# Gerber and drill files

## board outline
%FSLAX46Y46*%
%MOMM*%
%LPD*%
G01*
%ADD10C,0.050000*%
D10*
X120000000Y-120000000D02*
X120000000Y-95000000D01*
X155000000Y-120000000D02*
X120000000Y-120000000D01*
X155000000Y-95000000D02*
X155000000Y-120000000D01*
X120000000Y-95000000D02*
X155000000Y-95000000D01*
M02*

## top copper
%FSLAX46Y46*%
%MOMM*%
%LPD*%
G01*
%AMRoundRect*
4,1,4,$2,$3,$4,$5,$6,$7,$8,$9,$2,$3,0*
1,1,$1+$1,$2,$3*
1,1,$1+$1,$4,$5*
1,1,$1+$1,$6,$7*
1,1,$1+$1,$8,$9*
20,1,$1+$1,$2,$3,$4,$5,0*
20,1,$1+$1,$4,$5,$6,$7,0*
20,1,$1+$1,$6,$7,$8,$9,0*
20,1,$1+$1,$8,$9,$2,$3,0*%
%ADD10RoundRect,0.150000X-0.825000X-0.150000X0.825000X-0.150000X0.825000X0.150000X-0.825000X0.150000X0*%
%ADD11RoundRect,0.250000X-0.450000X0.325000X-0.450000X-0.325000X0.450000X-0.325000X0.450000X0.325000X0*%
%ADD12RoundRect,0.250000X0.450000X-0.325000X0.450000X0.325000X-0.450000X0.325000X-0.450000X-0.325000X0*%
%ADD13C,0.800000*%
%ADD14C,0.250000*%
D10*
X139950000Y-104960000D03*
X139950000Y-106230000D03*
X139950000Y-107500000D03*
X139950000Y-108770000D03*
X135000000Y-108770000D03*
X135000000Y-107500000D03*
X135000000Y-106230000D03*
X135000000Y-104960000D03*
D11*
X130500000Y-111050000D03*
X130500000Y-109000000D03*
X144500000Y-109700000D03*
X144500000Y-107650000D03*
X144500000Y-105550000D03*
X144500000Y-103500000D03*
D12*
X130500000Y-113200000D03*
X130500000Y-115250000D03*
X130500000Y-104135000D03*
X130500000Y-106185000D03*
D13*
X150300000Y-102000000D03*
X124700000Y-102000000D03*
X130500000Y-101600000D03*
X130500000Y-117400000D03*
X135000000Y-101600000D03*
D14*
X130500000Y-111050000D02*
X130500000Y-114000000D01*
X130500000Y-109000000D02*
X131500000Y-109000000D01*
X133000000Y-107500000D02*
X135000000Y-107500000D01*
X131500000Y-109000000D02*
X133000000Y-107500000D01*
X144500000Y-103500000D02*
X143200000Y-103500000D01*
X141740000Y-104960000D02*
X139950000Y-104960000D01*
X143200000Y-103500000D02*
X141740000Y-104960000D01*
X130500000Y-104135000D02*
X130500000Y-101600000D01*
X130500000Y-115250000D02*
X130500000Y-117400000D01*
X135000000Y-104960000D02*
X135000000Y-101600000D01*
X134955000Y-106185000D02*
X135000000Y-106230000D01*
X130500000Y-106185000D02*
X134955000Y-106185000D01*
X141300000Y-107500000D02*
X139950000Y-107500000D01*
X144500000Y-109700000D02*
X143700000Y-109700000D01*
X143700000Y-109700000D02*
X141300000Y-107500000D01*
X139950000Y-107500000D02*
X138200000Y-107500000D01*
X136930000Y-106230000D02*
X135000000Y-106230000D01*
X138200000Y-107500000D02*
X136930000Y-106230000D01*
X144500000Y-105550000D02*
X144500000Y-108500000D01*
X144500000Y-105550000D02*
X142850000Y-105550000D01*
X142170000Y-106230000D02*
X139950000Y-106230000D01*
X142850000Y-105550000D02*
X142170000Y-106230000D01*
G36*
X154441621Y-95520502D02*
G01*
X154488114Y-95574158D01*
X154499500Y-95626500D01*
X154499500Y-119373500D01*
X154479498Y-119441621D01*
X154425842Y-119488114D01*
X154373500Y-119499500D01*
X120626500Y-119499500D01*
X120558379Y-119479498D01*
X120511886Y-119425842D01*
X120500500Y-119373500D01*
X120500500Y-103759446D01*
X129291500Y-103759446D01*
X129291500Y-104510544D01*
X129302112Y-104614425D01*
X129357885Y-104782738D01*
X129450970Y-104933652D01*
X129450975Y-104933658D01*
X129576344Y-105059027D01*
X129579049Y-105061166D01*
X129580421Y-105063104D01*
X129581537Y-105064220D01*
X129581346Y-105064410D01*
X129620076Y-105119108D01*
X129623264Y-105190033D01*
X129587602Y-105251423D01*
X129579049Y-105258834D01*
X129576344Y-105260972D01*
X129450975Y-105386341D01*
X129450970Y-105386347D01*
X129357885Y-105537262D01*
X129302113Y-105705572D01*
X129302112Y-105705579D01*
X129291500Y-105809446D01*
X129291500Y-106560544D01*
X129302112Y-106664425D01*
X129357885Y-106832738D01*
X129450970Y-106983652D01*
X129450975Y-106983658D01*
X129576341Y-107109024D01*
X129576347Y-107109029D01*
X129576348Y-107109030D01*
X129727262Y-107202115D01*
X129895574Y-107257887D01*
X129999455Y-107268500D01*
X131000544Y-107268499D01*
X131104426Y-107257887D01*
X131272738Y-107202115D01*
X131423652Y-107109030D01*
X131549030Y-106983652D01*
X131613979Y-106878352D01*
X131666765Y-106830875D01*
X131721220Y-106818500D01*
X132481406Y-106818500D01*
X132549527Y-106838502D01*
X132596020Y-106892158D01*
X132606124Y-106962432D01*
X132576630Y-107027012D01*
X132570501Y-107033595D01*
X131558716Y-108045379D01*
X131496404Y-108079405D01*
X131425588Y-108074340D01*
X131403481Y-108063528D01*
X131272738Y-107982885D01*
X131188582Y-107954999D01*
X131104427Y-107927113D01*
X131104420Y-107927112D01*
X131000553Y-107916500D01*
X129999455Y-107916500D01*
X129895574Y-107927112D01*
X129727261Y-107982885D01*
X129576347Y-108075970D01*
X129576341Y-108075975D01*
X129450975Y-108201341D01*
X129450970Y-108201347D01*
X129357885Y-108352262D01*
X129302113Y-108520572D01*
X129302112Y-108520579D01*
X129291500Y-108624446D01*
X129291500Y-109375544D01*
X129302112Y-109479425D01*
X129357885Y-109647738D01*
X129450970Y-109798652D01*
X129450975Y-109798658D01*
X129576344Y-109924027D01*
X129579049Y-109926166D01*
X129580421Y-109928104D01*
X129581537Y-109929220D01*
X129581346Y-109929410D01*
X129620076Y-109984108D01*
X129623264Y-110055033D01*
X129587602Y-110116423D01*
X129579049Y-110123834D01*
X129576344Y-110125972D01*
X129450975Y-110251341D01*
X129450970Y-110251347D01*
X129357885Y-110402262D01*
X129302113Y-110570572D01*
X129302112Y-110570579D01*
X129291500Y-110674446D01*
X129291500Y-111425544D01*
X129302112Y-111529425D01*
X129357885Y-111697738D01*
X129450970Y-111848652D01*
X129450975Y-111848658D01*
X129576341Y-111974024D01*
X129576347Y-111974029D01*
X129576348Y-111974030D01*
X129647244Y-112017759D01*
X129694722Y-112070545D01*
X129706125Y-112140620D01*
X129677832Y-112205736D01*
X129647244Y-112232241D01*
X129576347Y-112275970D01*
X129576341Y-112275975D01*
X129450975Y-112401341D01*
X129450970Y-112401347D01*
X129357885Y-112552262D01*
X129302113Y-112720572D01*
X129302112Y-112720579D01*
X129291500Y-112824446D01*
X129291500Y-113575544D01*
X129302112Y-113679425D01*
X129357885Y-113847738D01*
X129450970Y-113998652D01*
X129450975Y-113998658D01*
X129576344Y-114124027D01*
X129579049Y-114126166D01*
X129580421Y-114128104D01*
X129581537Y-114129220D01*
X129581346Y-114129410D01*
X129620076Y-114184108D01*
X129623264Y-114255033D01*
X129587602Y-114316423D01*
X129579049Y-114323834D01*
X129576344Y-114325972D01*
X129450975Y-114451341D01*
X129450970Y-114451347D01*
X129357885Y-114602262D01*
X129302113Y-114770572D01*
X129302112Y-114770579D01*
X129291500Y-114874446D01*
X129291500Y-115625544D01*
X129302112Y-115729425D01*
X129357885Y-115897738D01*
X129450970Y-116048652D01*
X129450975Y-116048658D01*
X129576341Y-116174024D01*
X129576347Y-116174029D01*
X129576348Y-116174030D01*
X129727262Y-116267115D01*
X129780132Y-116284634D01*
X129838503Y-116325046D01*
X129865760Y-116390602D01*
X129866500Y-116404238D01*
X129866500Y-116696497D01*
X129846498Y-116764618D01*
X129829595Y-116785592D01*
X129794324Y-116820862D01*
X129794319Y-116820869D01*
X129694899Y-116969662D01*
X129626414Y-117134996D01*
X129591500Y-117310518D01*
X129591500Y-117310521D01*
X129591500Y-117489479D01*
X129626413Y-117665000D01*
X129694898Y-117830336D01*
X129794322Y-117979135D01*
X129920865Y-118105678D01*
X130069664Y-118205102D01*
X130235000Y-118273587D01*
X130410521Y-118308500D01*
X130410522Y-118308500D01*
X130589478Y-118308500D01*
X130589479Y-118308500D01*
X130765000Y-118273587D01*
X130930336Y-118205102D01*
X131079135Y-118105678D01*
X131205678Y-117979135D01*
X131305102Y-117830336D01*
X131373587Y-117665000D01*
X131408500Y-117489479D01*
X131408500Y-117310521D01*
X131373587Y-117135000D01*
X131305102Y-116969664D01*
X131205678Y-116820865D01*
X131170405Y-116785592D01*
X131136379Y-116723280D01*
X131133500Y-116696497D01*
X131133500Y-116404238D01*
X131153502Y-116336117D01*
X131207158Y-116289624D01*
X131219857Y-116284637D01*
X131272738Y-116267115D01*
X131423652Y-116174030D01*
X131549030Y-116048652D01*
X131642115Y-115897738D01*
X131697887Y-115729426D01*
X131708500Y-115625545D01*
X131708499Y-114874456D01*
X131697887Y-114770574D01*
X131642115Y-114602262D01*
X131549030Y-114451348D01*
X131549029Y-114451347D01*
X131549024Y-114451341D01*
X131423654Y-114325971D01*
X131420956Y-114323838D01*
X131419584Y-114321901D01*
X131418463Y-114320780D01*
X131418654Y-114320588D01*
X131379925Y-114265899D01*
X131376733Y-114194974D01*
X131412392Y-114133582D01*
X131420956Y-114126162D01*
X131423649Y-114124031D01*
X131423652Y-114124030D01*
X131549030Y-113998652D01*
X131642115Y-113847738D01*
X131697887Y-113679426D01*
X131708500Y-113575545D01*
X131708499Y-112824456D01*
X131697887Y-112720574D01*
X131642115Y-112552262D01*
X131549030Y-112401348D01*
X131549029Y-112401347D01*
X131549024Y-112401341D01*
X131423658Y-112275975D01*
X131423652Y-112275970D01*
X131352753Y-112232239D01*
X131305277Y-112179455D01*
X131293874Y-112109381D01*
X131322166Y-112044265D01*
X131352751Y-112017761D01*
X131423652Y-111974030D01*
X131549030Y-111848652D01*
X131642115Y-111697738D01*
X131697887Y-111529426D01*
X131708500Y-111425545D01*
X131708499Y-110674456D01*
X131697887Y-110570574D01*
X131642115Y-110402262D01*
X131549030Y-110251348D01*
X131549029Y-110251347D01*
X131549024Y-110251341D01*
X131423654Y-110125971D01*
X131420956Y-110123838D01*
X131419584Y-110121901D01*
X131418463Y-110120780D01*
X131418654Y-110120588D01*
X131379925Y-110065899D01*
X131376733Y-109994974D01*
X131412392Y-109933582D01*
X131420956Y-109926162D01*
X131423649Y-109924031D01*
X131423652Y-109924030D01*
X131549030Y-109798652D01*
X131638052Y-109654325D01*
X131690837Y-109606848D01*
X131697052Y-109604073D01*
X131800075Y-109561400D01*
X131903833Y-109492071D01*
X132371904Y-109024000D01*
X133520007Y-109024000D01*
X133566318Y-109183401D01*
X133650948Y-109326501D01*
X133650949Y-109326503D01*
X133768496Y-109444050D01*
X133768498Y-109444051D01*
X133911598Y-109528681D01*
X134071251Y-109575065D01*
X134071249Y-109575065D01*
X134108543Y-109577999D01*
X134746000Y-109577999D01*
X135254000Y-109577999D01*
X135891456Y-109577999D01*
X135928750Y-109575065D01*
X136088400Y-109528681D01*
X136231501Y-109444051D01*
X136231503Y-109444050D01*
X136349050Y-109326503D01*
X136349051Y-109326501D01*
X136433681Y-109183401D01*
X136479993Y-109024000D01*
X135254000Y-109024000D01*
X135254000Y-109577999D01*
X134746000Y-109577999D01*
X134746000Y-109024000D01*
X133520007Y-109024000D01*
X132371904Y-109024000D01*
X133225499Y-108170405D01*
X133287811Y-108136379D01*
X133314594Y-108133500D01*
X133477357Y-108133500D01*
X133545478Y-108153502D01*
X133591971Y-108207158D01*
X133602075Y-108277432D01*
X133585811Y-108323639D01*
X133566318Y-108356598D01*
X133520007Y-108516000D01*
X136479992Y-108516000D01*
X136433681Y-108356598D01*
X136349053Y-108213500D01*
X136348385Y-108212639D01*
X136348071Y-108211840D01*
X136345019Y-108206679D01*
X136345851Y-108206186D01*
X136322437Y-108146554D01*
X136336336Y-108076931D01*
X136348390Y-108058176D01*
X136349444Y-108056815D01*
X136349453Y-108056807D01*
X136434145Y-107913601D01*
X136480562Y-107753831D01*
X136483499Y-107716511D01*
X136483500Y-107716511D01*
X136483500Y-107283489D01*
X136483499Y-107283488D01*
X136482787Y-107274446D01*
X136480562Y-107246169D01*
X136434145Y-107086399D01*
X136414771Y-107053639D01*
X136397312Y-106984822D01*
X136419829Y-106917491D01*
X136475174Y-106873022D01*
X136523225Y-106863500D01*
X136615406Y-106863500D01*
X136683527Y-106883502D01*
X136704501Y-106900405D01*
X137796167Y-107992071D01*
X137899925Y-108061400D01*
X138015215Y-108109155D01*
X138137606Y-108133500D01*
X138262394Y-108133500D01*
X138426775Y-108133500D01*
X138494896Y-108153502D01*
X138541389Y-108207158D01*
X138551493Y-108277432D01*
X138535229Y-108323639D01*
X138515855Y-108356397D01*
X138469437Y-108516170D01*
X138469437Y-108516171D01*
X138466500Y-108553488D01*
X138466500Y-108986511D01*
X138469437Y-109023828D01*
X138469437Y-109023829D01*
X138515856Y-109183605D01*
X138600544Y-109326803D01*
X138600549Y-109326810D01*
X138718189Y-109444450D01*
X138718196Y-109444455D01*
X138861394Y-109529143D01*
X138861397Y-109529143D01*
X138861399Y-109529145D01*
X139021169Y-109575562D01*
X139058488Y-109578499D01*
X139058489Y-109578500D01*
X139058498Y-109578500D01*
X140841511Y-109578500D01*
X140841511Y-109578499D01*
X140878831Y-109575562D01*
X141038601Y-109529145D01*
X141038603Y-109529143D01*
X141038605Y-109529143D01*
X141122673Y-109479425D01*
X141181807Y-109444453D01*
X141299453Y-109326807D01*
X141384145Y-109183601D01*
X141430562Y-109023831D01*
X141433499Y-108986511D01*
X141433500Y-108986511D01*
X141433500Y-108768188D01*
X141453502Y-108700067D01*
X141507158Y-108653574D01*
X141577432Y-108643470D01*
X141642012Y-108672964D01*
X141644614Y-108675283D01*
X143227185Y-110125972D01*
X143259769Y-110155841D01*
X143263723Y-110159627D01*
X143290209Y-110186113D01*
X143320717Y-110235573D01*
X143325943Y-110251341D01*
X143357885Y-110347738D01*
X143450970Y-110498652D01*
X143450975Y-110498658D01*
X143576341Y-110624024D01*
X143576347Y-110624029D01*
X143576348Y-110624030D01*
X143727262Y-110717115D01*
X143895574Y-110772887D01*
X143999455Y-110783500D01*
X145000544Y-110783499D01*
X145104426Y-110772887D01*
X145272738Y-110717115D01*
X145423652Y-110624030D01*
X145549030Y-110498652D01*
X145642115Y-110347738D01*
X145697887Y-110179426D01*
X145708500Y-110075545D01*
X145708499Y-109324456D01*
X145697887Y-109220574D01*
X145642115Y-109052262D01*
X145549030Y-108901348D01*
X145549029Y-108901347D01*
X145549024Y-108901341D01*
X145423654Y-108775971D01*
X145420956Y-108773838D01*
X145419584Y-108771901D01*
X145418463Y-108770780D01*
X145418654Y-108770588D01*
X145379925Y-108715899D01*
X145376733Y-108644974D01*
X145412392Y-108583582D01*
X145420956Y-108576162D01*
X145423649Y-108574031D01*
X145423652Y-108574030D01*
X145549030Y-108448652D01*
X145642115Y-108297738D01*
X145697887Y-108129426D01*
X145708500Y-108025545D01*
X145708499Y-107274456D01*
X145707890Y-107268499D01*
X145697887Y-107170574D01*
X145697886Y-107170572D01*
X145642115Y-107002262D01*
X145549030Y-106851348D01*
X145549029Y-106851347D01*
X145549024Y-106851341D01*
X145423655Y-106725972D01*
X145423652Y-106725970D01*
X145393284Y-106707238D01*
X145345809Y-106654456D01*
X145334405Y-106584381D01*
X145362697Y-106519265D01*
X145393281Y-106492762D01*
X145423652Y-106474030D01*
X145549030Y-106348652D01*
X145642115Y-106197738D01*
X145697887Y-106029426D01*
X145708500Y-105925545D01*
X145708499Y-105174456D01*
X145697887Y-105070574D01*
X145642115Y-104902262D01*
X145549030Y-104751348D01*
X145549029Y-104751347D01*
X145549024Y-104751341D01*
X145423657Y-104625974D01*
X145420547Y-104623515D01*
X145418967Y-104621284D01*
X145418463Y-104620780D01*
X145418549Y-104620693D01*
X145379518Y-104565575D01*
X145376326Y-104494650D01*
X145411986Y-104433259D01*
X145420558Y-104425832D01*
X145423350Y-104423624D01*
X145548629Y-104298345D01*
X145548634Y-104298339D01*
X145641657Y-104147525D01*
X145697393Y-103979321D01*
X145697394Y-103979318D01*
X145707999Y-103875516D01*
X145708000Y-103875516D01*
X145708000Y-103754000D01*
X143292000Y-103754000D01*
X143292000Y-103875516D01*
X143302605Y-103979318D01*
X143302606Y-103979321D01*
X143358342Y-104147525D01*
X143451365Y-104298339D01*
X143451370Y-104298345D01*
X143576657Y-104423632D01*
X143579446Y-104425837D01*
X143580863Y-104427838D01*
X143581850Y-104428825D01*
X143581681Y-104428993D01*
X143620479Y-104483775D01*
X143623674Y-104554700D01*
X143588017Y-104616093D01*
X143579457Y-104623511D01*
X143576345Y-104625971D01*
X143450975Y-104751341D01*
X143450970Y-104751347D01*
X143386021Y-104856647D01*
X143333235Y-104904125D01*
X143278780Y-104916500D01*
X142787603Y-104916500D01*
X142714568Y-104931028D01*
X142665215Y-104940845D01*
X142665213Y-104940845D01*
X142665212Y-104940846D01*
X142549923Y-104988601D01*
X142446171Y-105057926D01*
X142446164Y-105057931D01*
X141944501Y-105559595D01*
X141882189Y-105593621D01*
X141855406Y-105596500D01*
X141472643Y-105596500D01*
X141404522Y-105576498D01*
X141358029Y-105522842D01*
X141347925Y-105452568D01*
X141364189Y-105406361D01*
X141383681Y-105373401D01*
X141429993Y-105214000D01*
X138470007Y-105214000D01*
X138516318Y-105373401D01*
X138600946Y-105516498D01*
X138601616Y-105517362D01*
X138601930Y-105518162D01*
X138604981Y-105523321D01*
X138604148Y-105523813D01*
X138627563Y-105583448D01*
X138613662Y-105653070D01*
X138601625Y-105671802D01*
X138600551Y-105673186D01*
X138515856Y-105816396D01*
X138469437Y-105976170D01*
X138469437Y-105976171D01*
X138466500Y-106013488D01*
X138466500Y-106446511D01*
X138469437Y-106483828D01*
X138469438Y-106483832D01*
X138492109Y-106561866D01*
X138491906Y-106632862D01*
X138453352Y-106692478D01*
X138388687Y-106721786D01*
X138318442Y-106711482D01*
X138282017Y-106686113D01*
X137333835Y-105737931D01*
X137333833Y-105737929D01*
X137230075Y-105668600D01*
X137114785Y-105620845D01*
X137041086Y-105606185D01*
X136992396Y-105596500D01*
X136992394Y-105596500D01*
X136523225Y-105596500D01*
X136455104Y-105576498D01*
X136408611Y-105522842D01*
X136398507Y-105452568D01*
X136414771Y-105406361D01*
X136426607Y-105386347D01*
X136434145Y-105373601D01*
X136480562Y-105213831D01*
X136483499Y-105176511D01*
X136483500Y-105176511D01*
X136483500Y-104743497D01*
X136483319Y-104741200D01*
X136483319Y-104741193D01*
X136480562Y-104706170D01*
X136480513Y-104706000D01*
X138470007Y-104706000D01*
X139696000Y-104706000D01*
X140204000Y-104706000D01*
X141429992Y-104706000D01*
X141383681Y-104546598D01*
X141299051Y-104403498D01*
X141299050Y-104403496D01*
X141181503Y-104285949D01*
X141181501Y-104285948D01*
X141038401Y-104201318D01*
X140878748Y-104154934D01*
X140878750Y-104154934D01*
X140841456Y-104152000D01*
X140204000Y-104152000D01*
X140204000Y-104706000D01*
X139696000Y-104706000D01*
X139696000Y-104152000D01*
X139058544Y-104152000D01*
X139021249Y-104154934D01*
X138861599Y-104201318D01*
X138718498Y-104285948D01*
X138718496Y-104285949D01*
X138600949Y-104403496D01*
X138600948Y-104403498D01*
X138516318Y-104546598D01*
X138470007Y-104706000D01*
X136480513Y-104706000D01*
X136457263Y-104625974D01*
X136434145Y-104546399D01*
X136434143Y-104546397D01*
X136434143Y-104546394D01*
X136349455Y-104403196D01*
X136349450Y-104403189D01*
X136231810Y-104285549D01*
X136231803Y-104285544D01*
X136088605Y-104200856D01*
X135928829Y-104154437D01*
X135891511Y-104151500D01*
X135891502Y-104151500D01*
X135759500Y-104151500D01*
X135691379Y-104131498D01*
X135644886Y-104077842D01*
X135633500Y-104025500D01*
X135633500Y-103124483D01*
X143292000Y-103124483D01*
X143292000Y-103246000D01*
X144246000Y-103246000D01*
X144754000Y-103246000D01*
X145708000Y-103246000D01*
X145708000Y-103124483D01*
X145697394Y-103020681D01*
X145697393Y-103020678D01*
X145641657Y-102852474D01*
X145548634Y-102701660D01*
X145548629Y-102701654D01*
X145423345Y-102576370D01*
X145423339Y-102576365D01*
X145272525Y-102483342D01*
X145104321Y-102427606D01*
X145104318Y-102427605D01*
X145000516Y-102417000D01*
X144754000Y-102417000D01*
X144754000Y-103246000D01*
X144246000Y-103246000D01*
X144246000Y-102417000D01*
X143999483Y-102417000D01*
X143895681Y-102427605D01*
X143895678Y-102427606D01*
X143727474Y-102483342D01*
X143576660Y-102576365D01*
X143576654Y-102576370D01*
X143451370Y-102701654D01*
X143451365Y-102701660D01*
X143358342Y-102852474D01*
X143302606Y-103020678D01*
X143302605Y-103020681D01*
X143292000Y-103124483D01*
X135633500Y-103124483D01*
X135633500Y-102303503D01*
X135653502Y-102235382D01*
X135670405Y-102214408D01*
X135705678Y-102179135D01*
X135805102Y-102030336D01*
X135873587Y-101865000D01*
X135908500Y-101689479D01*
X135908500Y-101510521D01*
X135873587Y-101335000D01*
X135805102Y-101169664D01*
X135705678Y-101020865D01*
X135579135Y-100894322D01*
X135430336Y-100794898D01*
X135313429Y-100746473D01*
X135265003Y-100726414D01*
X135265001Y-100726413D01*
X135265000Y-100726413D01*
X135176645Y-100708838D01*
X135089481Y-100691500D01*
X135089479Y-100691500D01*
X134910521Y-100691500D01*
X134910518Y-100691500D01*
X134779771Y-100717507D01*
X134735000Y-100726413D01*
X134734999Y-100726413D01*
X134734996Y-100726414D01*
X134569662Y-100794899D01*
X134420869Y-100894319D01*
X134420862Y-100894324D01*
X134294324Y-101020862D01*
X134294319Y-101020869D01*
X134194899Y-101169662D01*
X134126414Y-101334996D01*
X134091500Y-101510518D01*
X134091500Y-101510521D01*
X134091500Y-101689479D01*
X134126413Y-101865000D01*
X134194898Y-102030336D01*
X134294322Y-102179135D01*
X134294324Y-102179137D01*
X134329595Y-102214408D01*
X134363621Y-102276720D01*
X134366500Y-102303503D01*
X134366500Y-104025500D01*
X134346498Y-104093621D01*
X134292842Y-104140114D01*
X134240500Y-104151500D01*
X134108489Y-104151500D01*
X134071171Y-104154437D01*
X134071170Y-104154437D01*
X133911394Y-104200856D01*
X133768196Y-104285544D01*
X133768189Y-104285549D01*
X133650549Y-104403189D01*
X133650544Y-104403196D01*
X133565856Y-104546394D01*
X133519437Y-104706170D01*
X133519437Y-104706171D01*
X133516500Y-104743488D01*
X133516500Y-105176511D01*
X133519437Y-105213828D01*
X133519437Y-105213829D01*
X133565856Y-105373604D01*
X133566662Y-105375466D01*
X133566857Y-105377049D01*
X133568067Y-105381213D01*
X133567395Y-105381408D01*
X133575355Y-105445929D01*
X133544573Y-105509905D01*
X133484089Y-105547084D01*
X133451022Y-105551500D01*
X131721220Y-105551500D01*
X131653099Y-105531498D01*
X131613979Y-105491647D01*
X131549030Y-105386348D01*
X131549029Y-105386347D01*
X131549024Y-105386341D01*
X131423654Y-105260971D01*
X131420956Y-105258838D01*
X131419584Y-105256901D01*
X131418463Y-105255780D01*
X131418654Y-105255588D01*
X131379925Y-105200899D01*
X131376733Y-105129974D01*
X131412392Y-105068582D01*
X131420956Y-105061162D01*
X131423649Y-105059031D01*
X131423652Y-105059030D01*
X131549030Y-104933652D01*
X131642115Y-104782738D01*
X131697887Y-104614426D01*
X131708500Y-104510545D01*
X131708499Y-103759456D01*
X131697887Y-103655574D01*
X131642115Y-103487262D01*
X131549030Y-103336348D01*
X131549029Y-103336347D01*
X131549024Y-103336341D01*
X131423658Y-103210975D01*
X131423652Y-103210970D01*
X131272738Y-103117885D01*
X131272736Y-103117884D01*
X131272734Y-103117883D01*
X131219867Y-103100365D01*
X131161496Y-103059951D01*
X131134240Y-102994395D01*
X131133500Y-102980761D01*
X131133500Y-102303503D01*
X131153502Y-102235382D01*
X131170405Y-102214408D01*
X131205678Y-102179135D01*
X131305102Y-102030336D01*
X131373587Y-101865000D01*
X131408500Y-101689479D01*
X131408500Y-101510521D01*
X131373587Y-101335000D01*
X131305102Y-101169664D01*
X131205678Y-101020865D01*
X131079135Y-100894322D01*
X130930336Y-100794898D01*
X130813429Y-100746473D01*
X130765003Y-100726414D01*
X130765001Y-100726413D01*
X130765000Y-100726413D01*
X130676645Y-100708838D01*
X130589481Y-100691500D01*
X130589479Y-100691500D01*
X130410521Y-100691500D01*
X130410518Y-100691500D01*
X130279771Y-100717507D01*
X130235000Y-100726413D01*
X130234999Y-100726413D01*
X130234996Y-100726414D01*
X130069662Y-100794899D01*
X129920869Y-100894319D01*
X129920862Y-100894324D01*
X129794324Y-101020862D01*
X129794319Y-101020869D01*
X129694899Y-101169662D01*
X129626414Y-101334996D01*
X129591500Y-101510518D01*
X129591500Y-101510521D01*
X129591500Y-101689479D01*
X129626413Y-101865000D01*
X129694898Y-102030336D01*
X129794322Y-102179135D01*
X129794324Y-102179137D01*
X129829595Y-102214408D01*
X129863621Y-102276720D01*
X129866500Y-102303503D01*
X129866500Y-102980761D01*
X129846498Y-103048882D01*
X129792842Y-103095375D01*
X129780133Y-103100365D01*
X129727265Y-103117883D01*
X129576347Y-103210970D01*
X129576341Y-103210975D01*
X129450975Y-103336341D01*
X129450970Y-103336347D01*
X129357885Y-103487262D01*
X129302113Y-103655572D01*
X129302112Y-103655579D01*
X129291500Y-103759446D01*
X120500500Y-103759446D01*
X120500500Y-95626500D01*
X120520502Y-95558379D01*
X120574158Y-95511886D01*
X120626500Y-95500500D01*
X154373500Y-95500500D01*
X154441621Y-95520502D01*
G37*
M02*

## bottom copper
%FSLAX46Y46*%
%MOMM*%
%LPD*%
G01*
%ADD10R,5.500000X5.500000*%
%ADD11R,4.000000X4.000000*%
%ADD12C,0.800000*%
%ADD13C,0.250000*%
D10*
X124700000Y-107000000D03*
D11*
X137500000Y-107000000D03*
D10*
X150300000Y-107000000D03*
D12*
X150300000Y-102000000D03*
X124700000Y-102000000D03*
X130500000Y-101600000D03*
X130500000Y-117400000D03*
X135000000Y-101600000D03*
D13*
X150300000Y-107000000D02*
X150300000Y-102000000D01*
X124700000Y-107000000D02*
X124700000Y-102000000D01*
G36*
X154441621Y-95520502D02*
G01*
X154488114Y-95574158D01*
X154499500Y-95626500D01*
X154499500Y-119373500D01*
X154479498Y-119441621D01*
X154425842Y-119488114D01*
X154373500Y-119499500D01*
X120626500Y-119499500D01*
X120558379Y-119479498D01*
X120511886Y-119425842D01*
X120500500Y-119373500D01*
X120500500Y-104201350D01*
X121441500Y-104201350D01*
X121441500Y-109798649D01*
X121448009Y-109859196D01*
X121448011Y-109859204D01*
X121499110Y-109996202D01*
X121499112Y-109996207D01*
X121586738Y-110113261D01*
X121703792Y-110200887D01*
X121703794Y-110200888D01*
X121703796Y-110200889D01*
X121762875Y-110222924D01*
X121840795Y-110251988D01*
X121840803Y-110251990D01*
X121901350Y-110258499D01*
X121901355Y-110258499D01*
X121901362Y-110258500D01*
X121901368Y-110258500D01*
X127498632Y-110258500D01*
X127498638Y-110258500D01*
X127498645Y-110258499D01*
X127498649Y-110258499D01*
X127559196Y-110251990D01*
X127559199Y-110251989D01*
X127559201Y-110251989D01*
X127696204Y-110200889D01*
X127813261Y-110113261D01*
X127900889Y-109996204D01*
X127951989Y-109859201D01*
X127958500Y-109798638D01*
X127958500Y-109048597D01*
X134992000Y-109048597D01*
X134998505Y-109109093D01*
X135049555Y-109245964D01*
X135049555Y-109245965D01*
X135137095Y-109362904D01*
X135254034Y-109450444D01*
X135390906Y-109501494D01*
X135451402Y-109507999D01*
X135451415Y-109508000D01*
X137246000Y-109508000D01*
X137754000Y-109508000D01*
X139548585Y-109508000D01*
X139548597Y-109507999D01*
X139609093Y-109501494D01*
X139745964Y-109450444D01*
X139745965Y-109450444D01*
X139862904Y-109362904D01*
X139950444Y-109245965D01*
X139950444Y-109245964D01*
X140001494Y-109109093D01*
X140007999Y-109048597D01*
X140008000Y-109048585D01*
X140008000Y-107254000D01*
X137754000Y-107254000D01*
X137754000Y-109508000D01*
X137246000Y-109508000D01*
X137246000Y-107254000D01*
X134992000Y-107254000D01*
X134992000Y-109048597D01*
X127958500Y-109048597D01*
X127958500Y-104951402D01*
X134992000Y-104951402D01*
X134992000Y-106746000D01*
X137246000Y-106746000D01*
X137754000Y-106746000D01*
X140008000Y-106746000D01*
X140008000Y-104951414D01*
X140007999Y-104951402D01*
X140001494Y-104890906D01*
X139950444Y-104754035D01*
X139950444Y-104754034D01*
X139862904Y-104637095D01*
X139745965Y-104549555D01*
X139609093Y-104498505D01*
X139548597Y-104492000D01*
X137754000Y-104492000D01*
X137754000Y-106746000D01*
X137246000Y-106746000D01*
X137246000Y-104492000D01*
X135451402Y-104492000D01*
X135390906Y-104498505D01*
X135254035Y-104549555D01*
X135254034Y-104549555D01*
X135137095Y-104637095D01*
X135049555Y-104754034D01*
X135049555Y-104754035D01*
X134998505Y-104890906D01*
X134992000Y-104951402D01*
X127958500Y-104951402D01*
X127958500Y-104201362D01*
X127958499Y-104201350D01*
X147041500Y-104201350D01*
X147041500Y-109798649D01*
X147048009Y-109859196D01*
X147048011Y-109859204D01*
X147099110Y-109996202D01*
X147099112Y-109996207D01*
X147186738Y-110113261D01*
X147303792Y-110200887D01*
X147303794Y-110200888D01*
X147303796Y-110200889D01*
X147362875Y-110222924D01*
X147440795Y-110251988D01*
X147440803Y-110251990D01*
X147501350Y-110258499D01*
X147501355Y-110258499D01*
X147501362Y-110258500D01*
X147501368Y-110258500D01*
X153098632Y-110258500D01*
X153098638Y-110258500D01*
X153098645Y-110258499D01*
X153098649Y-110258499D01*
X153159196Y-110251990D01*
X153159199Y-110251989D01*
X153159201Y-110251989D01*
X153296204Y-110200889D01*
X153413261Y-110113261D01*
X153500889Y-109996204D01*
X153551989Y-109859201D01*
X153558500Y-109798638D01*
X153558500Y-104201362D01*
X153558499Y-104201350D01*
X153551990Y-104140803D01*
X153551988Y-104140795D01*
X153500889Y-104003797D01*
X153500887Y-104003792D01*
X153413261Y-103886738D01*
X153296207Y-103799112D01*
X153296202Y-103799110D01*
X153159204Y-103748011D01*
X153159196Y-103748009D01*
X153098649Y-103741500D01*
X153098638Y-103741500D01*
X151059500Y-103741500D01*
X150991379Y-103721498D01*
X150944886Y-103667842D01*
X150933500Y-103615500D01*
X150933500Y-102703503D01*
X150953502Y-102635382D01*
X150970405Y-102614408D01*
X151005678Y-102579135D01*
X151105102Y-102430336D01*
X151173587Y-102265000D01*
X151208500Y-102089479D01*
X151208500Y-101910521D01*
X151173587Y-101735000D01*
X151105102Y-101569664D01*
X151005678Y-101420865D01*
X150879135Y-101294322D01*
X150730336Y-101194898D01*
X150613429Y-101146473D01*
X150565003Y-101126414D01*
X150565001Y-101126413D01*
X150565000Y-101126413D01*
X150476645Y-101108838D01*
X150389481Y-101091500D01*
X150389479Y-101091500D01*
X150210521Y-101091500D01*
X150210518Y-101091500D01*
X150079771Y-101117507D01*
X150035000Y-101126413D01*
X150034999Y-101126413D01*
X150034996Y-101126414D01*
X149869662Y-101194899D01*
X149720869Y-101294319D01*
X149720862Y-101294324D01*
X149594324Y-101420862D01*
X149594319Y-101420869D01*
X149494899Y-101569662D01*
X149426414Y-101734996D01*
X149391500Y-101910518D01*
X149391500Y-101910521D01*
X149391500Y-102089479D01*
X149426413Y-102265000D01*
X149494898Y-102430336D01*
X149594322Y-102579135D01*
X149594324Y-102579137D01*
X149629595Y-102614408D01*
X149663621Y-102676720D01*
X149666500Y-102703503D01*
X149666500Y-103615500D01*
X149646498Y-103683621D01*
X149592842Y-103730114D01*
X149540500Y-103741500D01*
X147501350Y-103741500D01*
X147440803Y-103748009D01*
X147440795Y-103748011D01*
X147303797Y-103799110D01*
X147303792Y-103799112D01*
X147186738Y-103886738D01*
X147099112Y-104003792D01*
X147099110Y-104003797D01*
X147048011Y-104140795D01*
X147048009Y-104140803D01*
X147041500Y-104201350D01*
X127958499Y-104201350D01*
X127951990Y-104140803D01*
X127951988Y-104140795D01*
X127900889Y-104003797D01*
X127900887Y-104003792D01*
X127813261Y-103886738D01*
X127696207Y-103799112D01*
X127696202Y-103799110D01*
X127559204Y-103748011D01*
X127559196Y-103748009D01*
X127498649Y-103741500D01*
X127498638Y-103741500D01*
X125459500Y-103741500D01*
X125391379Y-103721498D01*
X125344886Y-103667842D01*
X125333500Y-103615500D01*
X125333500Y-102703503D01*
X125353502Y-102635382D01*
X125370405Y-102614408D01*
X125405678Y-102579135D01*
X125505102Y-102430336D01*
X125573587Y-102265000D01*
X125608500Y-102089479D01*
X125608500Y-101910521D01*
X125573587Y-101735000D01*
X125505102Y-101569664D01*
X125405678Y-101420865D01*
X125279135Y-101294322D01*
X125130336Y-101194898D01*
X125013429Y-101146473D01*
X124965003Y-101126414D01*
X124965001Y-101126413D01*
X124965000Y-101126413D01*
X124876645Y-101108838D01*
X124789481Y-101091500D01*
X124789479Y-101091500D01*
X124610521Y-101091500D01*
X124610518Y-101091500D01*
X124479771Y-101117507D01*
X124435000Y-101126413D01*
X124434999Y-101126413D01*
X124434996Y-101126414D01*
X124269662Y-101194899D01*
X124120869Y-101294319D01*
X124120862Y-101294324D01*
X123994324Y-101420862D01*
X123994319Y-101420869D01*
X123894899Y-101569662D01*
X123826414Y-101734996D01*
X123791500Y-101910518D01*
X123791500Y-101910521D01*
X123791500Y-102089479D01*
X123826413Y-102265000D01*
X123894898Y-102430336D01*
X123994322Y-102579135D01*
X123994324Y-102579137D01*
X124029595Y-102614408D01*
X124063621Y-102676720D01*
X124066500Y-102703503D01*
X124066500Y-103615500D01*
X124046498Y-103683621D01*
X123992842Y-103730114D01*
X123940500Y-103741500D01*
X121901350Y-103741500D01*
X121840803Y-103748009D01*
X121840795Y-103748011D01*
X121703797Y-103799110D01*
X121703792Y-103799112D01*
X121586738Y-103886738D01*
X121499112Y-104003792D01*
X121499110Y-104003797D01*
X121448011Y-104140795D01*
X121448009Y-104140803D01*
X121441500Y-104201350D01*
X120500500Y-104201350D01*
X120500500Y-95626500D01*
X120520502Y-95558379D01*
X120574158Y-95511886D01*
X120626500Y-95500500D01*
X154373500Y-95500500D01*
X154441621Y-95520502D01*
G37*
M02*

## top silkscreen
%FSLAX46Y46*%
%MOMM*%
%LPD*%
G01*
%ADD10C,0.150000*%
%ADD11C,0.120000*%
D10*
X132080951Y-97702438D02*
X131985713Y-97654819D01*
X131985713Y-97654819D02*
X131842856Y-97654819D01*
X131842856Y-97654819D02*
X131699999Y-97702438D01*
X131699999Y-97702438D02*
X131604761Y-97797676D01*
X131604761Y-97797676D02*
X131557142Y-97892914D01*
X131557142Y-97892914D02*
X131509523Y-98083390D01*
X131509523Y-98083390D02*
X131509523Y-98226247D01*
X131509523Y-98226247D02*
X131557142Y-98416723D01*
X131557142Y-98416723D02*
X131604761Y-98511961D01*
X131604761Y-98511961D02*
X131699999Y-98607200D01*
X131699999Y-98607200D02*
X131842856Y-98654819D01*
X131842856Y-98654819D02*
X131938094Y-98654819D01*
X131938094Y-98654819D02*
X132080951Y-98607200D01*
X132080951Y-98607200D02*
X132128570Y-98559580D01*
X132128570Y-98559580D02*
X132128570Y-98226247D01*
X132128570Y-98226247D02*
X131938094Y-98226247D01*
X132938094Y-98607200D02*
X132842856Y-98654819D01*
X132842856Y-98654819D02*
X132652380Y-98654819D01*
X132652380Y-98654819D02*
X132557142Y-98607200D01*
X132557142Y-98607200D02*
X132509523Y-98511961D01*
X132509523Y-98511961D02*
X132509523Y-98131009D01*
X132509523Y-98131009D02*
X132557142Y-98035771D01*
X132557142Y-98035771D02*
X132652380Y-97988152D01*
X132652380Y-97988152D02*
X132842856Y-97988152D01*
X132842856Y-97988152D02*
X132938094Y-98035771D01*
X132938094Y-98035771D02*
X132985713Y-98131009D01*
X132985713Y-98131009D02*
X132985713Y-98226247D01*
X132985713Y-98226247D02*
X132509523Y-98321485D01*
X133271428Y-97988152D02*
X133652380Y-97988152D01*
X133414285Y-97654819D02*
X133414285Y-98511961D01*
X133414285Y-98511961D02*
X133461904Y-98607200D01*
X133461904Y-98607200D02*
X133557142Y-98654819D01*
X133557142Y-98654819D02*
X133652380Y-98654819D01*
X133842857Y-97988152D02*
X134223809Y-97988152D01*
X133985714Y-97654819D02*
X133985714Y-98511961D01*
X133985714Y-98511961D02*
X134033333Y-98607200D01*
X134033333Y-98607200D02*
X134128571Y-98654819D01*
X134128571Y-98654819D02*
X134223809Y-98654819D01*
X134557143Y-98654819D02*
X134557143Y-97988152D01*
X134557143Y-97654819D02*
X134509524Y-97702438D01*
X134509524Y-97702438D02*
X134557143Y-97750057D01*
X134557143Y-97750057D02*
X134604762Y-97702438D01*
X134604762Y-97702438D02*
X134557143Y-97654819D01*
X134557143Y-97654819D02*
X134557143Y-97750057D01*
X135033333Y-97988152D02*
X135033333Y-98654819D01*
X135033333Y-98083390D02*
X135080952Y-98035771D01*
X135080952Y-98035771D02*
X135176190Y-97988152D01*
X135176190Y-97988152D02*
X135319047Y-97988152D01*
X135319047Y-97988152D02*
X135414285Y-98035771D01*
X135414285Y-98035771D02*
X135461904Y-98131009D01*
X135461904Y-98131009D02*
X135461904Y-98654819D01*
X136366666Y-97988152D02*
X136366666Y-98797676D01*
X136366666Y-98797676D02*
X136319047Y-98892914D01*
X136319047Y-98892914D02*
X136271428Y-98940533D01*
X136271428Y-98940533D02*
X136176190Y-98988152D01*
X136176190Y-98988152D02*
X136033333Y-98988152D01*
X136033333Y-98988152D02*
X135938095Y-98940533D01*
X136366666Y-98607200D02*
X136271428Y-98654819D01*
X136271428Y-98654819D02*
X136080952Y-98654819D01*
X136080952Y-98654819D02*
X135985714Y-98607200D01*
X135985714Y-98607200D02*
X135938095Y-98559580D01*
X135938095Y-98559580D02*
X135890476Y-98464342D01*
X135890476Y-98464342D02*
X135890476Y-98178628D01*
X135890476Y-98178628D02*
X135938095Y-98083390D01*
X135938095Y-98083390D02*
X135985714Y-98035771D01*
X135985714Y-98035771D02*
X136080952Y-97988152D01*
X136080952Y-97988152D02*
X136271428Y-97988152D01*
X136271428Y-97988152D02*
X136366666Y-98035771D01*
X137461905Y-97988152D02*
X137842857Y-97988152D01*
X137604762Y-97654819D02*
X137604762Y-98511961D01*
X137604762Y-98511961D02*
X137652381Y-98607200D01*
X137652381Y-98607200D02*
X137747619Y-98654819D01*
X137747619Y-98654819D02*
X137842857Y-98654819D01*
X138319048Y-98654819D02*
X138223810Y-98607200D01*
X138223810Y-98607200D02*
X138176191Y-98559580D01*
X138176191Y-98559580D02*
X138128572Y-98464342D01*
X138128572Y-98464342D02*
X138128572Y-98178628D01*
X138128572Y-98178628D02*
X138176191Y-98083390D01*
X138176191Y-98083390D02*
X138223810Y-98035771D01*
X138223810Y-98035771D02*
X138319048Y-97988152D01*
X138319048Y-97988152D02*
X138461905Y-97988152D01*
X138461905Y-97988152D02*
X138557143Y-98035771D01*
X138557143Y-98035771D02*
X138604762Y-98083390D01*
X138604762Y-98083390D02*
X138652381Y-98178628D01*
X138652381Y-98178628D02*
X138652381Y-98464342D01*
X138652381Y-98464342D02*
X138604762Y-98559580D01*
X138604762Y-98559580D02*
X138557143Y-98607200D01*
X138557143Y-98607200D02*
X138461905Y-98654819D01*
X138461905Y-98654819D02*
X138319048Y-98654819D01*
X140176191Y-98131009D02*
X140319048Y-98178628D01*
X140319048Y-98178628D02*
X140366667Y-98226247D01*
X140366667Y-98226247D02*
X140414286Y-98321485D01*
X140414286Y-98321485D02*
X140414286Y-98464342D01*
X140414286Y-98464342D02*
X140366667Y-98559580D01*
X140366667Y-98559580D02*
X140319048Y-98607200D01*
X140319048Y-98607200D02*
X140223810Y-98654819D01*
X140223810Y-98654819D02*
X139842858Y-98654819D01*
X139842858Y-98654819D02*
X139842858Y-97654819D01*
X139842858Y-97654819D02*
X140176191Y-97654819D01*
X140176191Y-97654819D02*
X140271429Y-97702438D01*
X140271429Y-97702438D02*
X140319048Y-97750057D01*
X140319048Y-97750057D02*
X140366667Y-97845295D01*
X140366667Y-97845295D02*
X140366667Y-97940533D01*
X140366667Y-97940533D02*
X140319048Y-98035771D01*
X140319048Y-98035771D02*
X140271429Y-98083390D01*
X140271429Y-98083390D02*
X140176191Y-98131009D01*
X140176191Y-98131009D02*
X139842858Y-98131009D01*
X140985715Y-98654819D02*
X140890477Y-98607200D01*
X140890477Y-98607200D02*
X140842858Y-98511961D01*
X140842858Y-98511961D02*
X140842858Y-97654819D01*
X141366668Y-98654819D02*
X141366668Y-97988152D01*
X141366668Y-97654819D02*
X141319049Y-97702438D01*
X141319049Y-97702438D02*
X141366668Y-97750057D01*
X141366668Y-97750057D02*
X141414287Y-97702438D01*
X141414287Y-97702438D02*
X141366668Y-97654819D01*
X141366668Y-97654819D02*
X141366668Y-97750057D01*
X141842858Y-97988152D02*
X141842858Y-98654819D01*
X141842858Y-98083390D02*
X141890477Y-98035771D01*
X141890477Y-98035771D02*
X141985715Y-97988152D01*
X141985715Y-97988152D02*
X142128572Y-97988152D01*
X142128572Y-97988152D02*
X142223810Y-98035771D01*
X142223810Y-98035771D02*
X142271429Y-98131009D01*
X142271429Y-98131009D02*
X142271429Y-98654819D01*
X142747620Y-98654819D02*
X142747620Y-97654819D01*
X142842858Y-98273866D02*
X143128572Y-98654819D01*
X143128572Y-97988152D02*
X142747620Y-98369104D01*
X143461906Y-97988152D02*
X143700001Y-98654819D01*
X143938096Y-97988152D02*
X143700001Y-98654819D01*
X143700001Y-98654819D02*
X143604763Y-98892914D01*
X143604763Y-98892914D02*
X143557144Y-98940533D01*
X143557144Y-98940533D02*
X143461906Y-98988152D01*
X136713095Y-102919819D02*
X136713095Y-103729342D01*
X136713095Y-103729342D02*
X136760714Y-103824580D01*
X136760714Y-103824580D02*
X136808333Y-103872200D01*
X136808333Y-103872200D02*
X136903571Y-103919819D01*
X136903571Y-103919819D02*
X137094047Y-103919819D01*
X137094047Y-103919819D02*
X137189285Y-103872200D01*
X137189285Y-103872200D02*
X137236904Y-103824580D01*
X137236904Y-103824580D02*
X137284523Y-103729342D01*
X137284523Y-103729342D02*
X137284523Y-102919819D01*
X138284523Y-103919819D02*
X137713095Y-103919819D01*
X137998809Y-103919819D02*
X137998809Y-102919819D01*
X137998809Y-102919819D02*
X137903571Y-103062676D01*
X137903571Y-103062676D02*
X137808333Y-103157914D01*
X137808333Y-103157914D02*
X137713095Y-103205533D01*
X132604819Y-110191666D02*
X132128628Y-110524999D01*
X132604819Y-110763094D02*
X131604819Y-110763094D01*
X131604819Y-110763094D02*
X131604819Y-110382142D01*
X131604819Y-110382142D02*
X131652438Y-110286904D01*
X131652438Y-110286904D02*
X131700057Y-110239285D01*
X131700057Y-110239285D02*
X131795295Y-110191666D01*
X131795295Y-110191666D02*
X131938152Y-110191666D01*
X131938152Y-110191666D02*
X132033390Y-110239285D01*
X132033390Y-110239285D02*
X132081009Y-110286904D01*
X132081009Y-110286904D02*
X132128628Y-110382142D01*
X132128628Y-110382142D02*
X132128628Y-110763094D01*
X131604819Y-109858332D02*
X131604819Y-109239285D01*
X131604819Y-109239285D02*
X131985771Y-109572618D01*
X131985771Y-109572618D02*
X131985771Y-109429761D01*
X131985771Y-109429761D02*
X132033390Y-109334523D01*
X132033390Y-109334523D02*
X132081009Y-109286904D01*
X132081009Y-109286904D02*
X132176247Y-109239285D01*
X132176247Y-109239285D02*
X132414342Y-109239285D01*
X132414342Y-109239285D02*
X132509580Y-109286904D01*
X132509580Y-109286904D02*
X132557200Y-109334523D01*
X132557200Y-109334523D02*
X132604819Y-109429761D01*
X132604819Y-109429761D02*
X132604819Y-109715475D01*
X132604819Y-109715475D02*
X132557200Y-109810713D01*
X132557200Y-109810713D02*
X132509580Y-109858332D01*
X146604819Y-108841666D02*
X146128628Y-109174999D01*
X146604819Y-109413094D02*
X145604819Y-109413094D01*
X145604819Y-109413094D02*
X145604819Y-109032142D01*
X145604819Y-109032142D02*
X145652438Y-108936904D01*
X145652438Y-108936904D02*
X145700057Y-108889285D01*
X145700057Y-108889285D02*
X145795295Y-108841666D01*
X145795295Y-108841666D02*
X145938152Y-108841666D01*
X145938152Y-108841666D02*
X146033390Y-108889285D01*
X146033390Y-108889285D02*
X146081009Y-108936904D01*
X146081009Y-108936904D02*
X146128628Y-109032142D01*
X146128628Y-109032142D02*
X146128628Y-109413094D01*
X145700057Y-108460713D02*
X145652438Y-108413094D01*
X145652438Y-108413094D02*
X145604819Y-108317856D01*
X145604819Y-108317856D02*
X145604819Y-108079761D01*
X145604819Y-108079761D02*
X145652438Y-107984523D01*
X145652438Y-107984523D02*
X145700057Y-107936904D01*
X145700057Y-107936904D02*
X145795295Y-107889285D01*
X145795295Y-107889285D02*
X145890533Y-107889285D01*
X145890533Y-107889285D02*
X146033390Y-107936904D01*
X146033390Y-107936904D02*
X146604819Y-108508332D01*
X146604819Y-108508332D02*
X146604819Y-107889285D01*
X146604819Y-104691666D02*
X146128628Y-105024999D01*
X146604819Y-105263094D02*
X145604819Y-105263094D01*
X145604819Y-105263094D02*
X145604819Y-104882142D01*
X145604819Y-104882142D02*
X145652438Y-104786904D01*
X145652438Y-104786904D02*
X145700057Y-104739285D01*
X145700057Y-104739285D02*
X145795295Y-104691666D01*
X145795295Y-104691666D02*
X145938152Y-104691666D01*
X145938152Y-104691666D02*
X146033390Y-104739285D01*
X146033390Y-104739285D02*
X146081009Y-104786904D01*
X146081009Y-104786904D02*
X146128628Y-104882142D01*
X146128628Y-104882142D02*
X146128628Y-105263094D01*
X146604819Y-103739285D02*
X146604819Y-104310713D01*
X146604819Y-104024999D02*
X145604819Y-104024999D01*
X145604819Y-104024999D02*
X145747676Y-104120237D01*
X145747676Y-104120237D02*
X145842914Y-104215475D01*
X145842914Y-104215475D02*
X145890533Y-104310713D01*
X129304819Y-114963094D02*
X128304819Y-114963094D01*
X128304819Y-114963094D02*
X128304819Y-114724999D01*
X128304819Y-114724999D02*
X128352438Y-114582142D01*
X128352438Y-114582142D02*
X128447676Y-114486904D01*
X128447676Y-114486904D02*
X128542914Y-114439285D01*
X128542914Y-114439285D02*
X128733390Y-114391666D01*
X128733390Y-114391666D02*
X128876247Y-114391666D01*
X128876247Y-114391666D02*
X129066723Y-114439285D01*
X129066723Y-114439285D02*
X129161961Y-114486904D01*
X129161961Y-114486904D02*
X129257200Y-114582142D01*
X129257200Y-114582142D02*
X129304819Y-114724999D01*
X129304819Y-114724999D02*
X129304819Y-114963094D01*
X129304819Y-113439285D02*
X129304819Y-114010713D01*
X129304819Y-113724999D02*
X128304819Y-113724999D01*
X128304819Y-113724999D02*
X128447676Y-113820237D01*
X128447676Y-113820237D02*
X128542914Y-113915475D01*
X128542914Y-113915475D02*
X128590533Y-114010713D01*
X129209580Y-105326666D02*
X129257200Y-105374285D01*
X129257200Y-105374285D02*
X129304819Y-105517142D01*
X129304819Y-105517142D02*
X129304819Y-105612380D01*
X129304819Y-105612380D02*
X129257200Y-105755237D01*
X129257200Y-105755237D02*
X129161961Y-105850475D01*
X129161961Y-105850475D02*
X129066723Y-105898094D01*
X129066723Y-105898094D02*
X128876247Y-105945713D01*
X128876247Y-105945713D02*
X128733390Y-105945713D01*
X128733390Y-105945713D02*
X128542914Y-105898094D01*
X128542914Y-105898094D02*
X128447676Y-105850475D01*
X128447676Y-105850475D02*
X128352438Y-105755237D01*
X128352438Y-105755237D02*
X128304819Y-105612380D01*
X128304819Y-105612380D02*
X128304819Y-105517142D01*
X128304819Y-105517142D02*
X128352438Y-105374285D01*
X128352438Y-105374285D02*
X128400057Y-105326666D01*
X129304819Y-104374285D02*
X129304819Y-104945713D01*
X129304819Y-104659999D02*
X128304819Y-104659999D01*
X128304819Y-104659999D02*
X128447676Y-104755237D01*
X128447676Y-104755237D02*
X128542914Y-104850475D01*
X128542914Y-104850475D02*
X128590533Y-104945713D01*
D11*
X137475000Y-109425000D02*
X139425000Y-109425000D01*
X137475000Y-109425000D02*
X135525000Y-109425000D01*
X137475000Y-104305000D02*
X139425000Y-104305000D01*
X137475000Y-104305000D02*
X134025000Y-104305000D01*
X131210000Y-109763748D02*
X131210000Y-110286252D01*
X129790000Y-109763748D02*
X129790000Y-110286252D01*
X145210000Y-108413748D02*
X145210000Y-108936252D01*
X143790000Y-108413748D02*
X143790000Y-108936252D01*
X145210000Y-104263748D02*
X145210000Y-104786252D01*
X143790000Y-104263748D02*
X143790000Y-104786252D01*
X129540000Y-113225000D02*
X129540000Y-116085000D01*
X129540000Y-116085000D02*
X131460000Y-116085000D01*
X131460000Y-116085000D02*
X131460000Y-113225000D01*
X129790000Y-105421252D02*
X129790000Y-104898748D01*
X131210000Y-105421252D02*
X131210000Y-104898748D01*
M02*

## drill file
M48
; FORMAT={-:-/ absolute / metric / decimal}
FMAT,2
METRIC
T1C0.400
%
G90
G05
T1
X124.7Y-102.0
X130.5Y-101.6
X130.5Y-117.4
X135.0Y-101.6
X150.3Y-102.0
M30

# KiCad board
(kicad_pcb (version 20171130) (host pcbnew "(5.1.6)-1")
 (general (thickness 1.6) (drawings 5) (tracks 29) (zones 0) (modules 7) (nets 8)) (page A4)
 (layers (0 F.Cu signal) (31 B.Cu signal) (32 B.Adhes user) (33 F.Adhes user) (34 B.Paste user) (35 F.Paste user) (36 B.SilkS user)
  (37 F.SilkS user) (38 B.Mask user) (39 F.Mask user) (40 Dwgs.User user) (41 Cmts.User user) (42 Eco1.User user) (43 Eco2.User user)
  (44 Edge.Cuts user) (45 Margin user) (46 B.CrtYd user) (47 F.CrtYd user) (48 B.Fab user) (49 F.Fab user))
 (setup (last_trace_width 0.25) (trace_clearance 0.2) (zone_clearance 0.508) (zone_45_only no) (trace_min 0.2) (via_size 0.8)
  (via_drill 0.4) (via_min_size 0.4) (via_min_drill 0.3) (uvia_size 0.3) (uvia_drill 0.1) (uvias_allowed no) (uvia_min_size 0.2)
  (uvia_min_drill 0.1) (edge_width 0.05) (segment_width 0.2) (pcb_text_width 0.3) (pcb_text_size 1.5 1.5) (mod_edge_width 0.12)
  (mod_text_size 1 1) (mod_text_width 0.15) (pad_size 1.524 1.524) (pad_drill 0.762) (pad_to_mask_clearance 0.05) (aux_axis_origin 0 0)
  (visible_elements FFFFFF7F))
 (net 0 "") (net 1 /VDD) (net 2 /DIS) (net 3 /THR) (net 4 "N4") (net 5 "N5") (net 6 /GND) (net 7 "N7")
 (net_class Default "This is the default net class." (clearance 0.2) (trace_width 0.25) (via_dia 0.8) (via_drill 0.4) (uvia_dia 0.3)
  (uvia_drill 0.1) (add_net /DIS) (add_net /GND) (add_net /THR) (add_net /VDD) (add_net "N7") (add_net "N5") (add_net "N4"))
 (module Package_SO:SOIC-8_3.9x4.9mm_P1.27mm (layer F.Cu) (at 137.475 106.865)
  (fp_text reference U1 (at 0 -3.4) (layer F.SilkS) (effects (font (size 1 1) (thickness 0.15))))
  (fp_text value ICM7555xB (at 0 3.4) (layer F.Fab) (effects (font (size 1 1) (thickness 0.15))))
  (fp_line (start 0 2.56) (end 1.95 2.56) (layer F.SilkS) (width 0.12))
  (fp_line (start 0 2.56) (end -1.95 2.56) (layer F.SilkS) (width 0.12))
  (fp_line (start 0 -2.56) (end 1.95 -2.56) (layer F.SilkS) (width 0.12))
  (fp_line (start 0 -2.56) (end -3.45 -2.56) (layer F.SilkS) (width 0.12))
  (pad 8 smd roundrect (at 2.475 -1.905) (size 1.95 0.6) (layers F.Cu F.Paste F.Mask) (roundrect_rratio 0.25) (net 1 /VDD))
  (pad 7 smd roundrect (at 2.475 -0.635) (size 1.95 0.6) (layers F.Cu F.Paste F.Mask) (roundrect_rratio 0.25) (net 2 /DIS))
  (pad 6 smd roundrect (at 2.475 0.635) (size 1.95 0.6) (layers F.Cu F.Paste F.Mask) (roundrect_rratio 0.25) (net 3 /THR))
  (pad 5 smd roundrect (at 2.475 1.905) (size 1.95 0.6) (layers F.Cu F.Paste F.Mask) (roundrect_rratio 0.25) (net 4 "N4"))
  (pad 4 smd roundrect (at -2.475 1.905) (size 1.95 0.6) (layers F.Cu F.Paste F.Mask) (roundrect_rratio 0.25) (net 1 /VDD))
  (pad 3 smd roundrect (at -2.475 0.635) (size 1.95 0.6) (layers F.Cu F.Paste F.Mask) (roundrect_rratio 0.25) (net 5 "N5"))
  (pad 2 smd roundrect (at -2.475 -0.635) (size 1.95 0.6) (layers F.Cu F.Paste F.Mask) (roundrect_rratio 0.25) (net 3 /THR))
  (pad 1 smd roundrect (at -2.475 -1.905) (size 1.95 0.6) (layers F.Cu F.Paste F.Mask) (roundrect_rratio 0.25) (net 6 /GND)))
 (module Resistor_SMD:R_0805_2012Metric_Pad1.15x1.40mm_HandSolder (layer F.Cu) (at 130.5 110.025 270)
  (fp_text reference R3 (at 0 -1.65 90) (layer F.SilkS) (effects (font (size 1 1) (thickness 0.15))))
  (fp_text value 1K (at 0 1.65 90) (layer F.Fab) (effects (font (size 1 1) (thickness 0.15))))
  (fp_line (start -0.261252 -0.71) (end 0.261252 -0.71) (layer F.SilkS) (width 0.12))
  (fp_line (start -0.261252 0.71) (end 0.261252 0.71) (layer F.SilkS) (width 0.12))
  (pad 2 smd roundrect (at 1.025 0 270) (size 1.15 1.4) (layers F.Cu F.Paste F.Mask) (roundrect_rratio 0.217391) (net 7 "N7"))
  (pad 1 smd roundrect (at -1.025 0 270) (size 1.15 1.4) (layers F.Cu F.Paste F.Mask) (roundrect_rratio 0.217391) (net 5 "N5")))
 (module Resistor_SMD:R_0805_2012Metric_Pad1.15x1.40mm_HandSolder (layer F.Cu) (at 144.5 108.675 270)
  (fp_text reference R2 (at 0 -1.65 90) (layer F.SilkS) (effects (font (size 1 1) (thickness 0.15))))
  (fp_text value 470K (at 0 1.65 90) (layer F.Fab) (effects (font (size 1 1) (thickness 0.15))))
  (fp_line (start -0.261252 -0.71) (end 0.261252 -0.71) (layer F.SilkS) (width 0.12))
  (fp_line (start -0.261252 0.71) (end 0.261252 0.71) (layer F.SilkS) (width 0.12))
  (pad 2 smd roundrect (at 1.025 0 270) (size 1.15 1.4) (layers F.Cu F.Paste F.Mask) (roundrect_rratio 0.217391) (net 3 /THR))
  (pad 1 smd roundrect (at -1.025 0 270) (size 1.15 1.4) (layers F.Cu F.Paste F.Mask) (roundrect_rratio 0.217391) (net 2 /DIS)))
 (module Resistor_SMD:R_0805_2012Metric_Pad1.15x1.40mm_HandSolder (layer F.Cu) (at 144.5 104.525 270)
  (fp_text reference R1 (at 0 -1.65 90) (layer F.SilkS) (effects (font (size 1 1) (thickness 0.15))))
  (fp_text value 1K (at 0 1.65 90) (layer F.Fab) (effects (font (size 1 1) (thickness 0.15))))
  (fp_line (start -0.261252 -0.71) (end 0.261252 -0.71) (layer F.SilkS) (width 0.12))
  (fp_line (start -0.261252 0.71) (end 0.261252 0.71) (layer F.SilkS) (width 0.12))
  (pad 2 smd roundrect (at 1.025 0 270) (size 1.15 1.4) (layers F.Cu F.Paste F.Mask) (roundrect_rratio 0.217391) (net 2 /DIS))
  (pad 1 smd roundrect (at -1.025 0 270) (size 1.15 1.4) (layers F.Cu F.Paste F.Mask) (roundrect_rratio 0.217391) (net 1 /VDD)))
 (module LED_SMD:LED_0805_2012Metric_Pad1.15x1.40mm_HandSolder (layer F.Cu) (at 130.5 114.225 90)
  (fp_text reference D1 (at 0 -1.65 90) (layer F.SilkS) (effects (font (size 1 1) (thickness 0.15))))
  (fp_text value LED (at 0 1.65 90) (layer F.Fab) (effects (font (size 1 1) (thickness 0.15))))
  (fp_line (start 1 -0.96) (end -1.86 -0.96) (layer F.SilkS) (width 0.12))
  (fp_line (start -1.86 -0.96) (end -1.86 0.96) (layer F.SilkS) (width 0.12))
  (fp_line (start -1.86 0.96) (end 1 0.96) (layer F.SilkS) (width 0.12))
  (pad 2 smd roundrect (at 1.025 0 90) (size 1.15 1.4) (layers F.Cu F.Paste F.Mask) (roundrect_rratio 0.217391) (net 7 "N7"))
  (pad 1 smd roundrect (at -1.025 0 90) (size 1.15 1.4) (layers F.Cu F.Paste F.Mask) (roundrect_rratio 0.217391) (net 6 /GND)))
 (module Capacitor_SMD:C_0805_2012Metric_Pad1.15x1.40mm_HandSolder (layer F.Cu) (at 130.5 105.16 90)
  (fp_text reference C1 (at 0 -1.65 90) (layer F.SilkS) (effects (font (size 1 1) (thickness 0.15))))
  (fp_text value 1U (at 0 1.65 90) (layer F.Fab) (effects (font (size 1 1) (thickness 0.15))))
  (fp_line (start -0.261252 -0.71) (end 0.261252 -0.71) (layer F.SilkS) (width 0.12))
  (fp_line (start -0.261252 0.71) (end 0.261252 0.71) (layer F.SilkS) (width 0.12))
  (pad 2 smd roundrect (at 1.025 0 90) (size 1.15 1.4) (layers F.Cu F.Paste F.Mask) (roundrect_rratio 0.217391) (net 6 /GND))
  (pad 1 smd roundrect (at -1.025 0 90) (size 1.15 1.4) (layers F.Cu F.Paste F.Mask) (roundrect_rratio 0.217391) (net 3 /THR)))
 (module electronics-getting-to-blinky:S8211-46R (layer B.Cu) (at 137.5 107)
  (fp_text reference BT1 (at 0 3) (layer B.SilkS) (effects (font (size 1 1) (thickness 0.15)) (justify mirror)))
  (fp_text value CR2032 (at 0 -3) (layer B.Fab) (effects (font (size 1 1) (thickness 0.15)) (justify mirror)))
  (pad 1 smd rect (at -12.8 0) (size 5.5 5.5) (layers B.Cu B.Paste B.Mask) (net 1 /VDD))
  (pad 2 smd rect (at 0 0) (size 4 4) (layers B.Cu B.Paste B.Mask) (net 6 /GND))
  (pad 1 smd rect (at 12.8 0) (size 5.5 5.5) (layers B.Cu B.Paste B.Mask) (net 1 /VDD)))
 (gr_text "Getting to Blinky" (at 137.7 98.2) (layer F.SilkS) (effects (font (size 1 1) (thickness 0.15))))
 (gr_line (start 120 120) (end 120 95) (layer Edge.Cuts) (width 0.05))
 (gr_line (start 155 120) (end 120 120) (layer Edge.Cuts) (width 0.05))
 (gr_line (start 155 95) (end 155 120) (layer Edge.Cuts) (width 0.05))
 (gr_line (start 120 95) (end 155 95) (layer Edge.Cuts) (width 0.05))
 (segment (start 130.5 111.05) (end 130.5 114) (width 0.25) (layer F.Cu) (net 7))
 (segment (start 130.5 109) (end 131.5 109) (width 0.25) (layer F.Cu) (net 5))
 (segment (start 133 107.5) (end 135 107.5) (width 0.25) (layer F.Cu) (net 5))
 (segment (start 131.5 109) (end 133 107.5) (width 0.25) (layer F.Cu) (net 5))
 (segment (start 144.5 103.5) (end 143.2 103.5) (width 0.25) (layer F.Cu) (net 1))
 (segment (start 141.74 104.96) (end 139.95 104.96) (width 0.25) (layer F.Cu) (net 1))
 (segment (start 143.2 103.5) (end 141.74 104.96) (width 0.25) (layer F.Cu) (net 1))
 (via (at 150.3 102) (size 0.8) (drill 0.4) (layers F.Cu B.Cu) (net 1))
 (segment (start 150.3 107) (end 150.3 102) (width 0.25) (layer B.Cu) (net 1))
 (via (at 124.7 102) (size 0.8) (drill 0.4) (layers F.Cu B.Cu) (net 1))
 (segment (start 124.7 107) (end 124.7 102) (width 0.25) (layer B.Cu) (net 1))
 (via (at 130.5 101.6) (size 0.8) (drill 0.4) (layers F.Cu B.Cu) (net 6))
 (segment (start 130.5 104.135) (end 130.5 101.6) (width 0.25) (layer F.Cu) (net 6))
 (via (at 130.5 117.4) (size 0.8) (drill 0.4) (layers F.Cu B.Cu) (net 6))
 (segment (start 130.5 115.25) (end 130.5 117.4) (width 0.25) (layer F.Cu) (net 6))
 (via (at 135 101.6) (size 0.8) (drill 0.4) (layers F.Cu B.Cu) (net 6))
 (segment (start 135 104.96) (end 135 101.6) (width 0.25) (layer F.Cu) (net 6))
 (segment (start 134.955 106.185) (end 135 106.23) (width 0.25) (layer F.Cu) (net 3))
 (segment (start 130.5 106.185) (end 134.955 106.185) (width 0.25) (layer F.Cu) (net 3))
 (segment (start 141.3 107.5) (end 139.95 107.5) (width 0.25) (layer F.Cu) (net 3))
 (segment (start 144.5 109.7) (end 143.7 109.7) (width 0.25) (layer F.Cu) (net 3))
 (segment (start 143.7 109.7) (end 141.3 107.5) (width 0.25) (layer F.Cu) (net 3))
 (segment (start 139.95 107.5) (end 138.2 107.5) (width 0.25) (layer F.Cu) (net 3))
 (segment (start 136.93 106.23) (end 135 106.23) (width 0.25) (layer F.Cu) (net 3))
 (segment (start 138.2 107.5) (end 136.93 106.23) (width 0.25) (layer F.Cu) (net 3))
 (segment (start 144.5 105.55) (end 144.5 108.5) (width 0.25) (layer F.Cu) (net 2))
 (segment (start 144.5 105.55) (end 142.85 105.55) (width 0.25) (layer F.Cu) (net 2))
 (segment (start 142.17 106.23) (end 139.95 106.23) (width 0.25) (layer F.Cu) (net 2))
 (segment (start 142.85 105.55) (end 142.17 106.23) (width 0.25) (layer F.Cu) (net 2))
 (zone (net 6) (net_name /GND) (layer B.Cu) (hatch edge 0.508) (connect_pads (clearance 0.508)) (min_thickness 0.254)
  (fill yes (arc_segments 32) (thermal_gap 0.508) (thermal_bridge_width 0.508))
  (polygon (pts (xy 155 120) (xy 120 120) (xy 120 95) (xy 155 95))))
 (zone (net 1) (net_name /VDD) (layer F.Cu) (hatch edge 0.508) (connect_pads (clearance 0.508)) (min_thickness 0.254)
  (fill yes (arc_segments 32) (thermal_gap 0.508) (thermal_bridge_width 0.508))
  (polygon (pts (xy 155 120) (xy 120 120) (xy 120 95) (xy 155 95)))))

